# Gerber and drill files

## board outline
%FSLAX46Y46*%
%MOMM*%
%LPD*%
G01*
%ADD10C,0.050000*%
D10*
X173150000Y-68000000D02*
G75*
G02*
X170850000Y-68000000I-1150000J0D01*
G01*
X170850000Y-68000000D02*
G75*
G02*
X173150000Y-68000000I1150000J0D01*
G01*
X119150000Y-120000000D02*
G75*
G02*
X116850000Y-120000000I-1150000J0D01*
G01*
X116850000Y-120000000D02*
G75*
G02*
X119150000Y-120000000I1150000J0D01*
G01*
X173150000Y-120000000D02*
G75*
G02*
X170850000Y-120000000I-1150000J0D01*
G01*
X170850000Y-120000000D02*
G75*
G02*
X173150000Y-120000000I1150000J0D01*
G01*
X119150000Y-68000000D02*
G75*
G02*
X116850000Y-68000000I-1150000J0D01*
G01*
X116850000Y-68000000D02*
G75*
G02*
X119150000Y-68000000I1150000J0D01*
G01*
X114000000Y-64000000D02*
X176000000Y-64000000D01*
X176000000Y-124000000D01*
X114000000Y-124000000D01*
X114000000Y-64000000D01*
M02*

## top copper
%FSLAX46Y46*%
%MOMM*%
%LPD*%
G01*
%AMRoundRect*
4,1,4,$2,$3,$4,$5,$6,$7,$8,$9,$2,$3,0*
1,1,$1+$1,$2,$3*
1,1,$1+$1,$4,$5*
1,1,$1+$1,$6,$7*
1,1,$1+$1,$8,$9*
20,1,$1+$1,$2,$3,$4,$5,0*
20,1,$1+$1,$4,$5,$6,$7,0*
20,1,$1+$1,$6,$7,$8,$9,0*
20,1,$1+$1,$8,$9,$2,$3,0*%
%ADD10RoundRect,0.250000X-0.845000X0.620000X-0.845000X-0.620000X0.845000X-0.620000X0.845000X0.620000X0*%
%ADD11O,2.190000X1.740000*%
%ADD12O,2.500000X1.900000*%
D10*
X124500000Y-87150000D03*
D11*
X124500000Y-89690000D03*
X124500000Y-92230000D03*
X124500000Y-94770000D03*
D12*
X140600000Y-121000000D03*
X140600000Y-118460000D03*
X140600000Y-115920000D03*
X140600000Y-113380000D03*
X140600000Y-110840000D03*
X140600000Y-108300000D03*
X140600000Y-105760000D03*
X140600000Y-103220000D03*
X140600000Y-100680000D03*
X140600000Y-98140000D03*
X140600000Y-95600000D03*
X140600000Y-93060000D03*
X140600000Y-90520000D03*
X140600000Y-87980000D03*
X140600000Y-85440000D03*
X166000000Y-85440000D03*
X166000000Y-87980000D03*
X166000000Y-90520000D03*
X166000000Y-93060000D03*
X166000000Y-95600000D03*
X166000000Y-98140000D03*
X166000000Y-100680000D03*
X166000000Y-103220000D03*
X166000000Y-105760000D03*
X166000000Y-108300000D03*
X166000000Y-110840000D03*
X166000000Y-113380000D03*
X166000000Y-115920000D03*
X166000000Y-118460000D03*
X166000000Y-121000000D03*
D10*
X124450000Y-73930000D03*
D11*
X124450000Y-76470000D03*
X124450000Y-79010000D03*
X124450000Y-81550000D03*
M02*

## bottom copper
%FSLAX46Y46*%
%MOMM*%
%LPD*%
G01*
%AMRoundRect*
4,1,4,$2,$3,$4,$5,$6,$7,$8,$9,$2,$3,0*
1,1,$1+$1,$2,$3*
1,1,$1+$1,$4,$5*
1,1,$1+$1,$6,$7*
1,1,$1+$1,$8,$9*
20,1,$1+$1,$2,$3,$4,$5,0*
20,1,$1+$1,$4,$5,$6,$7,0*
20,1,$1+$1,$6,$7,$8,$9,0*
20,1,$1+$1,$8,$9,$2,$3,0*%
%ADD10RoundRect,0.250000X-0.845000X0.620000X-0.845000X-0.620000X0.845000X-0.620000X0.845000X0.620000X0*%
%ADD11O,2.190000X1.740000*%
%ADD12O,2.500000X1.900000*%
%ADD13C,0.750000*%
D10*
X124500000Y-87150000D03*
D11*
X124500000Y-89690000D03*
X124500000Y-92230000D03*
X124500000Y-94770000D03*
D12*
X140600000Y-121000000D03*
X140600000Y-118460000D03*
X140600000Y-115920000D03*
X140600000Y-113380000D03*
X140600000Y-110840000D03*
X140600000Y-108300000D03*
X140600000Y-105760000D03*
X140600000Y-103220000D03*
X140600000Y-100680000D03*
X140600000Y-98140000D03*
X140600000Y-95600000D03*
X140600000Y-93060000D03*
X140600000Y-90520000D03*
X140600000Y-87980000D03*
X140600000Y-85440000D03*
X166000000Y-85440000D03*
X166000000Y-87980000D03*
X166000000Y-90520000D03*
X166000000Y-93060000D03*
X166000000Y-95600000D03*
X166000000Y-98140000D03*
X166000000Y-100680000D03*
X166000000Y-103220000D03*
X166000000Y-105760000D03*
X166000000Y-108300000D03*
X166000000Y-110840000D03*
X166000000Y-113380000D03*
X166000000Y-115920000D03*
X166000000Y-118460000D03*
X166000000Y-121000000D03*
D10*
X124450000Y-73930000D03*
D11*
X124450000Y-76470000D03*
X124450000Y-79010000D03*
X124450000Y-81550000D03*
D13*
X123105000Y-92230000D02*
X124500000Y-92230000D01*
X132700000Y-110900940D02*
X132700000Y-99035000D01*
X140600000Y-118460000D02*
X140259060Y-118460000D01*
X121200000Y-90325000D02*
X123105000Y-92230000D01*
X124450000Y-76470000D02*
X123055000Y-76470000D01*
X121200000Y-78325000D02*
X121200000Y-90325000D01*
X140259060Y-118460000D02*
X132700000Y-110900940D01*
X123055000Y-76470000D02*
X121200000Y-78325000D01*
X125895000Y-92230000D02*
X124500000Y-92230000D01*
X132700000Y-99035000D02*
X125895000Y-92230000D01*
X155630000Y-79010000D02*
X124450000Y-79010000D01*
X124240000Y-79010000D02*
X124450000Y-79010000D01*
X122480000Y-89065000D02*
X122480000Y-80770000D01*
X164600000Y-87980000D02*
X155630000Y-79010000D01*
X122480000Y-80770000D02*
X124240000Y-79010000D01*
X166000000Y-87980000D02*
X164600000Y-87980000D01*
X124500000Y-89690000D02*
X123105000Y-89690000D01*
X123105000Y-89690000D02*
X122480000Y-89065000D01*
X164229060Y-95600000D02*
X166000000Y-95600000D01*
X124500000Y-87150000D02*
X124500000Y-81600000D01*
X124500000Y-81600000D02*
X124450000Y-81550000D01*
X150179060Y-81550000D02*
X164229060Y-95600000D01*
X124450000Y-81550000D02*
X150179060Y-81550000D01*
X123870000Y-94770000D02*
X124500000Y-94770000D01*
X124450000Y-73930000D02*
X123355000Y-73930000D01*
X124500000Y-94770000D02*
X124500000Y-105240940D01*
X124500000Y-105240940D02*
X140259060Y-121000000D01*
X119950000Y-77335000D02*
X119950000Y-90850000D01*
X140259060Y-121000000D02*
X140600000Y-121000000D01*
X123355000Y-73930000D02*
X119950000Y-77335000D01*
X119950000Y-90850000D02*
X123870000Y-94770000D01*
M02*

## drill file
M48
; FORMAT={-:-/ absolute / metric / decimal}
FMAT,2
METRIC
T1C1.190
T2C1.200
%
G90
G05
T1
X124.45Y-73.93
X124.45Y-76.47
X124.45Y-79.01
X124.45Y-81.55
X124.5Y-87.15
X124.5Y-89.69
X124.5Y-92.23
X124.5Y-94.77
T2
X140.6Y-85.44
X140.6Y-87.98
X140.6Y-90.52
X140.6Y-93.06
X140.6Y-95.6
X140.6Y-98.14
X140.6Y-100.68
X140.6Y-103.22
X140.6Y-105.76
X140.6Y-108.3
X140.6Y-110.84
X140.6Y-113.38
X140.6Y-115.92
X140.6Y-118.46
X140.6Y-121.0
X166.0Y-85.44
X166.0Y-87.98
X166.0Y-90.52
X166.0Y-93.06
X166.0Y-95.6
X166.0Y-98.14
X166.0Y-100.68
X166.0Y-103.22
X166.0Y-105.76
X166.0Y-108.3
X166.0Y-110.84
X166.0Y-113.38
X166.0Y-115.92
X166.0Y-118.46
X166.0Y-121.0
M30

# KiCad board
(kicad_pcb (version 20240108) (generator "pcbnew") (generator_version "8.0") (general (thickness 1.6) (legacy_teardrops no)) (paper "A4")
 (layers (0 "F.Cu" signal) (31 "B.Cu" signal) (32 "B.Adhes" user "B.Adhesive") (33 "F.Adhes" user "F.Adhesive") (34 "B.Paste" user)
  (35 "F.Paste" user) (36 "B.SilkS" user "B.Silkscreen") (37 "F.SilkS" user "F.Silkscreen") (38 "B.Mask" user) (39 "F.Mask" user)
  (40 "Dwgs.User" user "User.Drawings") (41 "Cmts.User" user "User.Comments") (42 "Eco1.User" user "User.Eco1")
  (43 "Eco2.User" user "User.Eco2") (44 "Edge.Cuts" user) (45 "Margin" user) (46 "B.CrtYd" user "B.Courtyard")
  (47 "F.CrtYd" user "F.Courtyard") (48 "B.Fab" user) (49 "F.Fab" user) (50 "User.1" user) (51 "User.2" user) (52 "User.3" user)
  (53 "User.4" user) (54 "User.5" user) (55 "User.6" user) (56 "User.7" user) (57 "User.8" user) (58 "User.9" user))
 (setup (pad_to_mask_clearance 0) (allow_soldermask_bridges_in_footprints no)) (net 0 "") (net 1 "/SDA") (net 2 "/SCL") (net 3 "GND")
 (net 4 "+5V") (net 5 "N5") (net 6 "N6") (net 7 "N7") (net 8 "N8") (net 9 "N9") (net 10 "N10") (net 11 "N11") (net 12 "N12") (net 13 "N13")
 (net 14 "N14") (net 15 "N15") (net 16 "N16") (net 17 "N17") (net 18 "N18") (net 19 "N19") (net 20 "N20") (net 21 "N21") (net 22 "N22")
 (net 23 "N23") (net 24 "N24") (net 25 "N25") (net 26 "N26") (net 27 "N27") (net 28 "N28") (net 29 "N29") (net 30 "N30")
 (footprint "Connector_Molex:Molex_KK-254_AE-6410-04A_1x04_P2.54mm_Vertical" (layer "F.Cu") (at 124.5 87.15 -90)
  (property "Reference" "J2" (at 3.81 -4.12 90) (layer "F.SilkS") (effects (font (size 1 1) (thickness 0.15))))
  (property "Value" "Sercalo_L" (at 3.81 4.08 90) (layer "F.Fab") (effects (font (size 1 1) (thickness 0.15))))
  (pad "1" thru_hole roundrect (at 0 0 270) (size 1.74 2.19) (drill 1.19) (layers "*.Cu" "*.Mask") (remove_unused_layers no)
   (roundrect_rratio 0.143678) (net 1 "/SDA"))
  (pad "2" thru_hole oval (at 2.54 0 270) (size 1.74 2.19) (drill 1.19) (layers "*.Cu" "*.Mask") (remove_unused_layers no) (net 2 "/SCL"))
  (pad "3" thru_hole oval (at 5.08 0 270) (size 1.74 2.19) (drill 1.19) (layers "*.Cu" "*.Mask") (remove_unused_layers no) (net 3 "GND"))
  (pad "4" thru_hole oval (at 7.62 0 270) (size 1.74 2.19) (drill 1.19) (layers "*.Cu" "*.Mask") (remove_unused_layers no) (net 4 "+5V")))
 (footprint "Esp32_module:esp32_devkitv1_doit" (layer "F.Cu") (at 153.3 104.49)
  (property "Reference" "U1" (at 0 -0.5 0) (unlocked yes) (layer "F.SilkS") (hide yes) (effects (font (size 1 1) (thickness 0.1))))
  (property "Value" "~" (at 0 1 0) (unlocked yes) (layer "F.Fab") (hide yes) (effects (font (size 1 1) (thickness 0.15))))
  (pad "1" thru_hole oval (at -12.7 16.51 180) (size 2.5 1.9) (drill 1.2) (layers "*.Cu" "*.Mask") (remove_unused_layers no) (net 4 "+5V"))
  (pad "2" thru_hole oval (at -12.7 13.97 180) (size 2.5 1.9) (drill 1.2) (layers "*.Cu" "*.Mask") (remove_unused_layers no) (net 3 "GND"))
  (pad "3" thru_hole oval (at -12.7 11.43 180) (size 2.5 1.9) (drill 1.2) (layers "*.Cu" "*.Mask") (remove_unused_layers no) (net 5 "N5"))
  (pad "4" thru_hole oval (at -12.7 8.89 180) (size 2.5 1.9) (drill 1.2) (layers "*.Cu" "*.Mask") (remove_unused_layers no) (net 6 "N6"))
  (pad "5" thru_hole oval (at -12.7 6.35 180) (size 2.5 1.9) (drill 1.2) (layers "*.Cu" "*.Mask") (remove_unused_layers no) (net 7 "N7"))
  (pad "6" thru_hole oval (at -12.7 3.81 180) (size 2.5 1.9) (drill 1.2) (layers "*.Cu" "*.Mask") (remove_unused_layers no) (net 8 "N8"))
  (pad "7" thru_hole oval (at -12.7 1.27 180) (size 2.5 1.9) (drill 1.2) (layers "*.Cu" "*.Mask") (remove_unused_layers no) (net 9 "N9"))
  (pad "8" thru_hole oval (at -12.7 -1.27 180) (size 2.5 1.9) (drill 1.2) (layers "*.Cu" "*.Mask") (remove_unused_layers no) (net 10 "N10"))
  (pad "9" thru_hole oval (at -12.7 -3.81 180) (size 2.5 1.9) (drill 1.2) (layers "*.Cu" "*.Mask") (remove_unused_layers no) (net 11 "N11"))
  (pad "10" thru_hole oval (at -12.7 -6.35 180) (size 2.5 1.9) (drill 1.2) (layers "*.Cu" "*.Mask") (remove_unused_layers no) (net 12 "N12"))
  (pad "11" thru_hole oval (at -12.7 -8.89 180) (size 2.5 1.9) (drill 1.2) (layers "*.Cu" "*.Mask") (remove_unused_layers no) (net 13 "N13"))
  (pad "12" thru_hole oval (at -12.7 -11.43 180) (size 2.5 1.9) (drill 1.2) (layers "*.Cu" "*.Mask") (remove_unused_layers no)
   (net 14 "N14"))
  (pad "13" thru_hole oval (at -12.7 -13.97 180) (size 2.5 1.9) (drill 1.2) (layers "*.Cu" "*.Mask") (remove_unused_layers no)
   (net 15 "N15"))
  (pad "14" thru_hole oval (at -12.7 -16.51 180) (size 2.5 1.9) (drill 1.2) (layers "*.Cu" "*.Mask") (remove_unused_layers no)
   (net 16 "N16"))
  (pad "15" thru_hole oval (at -12.7 -19.05 180) (size 2.5 1.9) (drill 1.2) (layers "*.Cu" "*.Mask") (remove_unused_layers no)
   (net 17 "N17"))
  (pad "16" thru_hole oval (at 12.7 -19.05 180) (size 2.5 1.9) (drill 1.2) (layers "*.Cu" "*.Mask") (remove_unused_layers no) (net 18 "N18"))
  (pad "17" thru_hole oval (at 12.7 -16.51 180) (size 2.5 1.9) (drill 1.2) (layers "*.Cu" "*.Mask") (remove_unused_layers no) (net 2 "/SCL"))
  (pad "18" thru_hole oval (at 12.7 -13.97 180) (size 2.5 1.9) (drill 1.2) (layers "*.Cu" "*.Mask") (remove_unused_layers no) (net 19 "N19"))
  (pad "19" thru_hole oval (at 12.7 -11.43 180) (size 2.5 1.9) (drill 1.2) (layers "*.Cu" "*.Mask") (remove_unused_layers no) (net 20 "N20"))
  (pad "20" thru_hole oval (at 12.7 -8.89 180) (size 2.5 1.9) (drill 1.2) (layers "*.Cu" "*.Mask") (remove_unused_layers no) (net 1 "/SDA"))
  (pad "21" thru_hole oval (at 12.7 -6.35 180) (size 2.5 1.9) (drill 1.2) (layers "*.Cu" "*.Mask") (remove_unused_layers no) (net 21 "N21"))
  (pad "22" thru_hole oval (at 12.7 -3.81 180) (size 2.5 1.9) (drill 1.2) (layers "*.Cu" "*.Mask") (remove_unused_layers no) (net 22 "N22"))
  (pad "23" thru_hole oval (at 12.7 -1.27 180) (size 2.5 1.9) (drill 1.2) (layers "*.Cu" "*.Mask") (remove_unused_layers no) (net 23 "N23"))
  (pad "24" thru_hole oval (at 12.7 1.27 180) (size 2.5 1.9) (drill 1.2) (layers "*.Cu" "*.Mask") (remove_unused_layers no) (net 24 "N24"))
  (pad "25" thru_hole oval (at 12.7 3.81 180) (size 2.5 1.9) (drill 1.2) (layers "*.Cu" "*.Mask") (remove_unused_layers no) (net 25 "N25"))
  (pad "26" thru_hole oval (at 12.7 6.35 180) (size 2.5 1.9) (drill 1.2) (layers "*.Cu" "*.Mask") (remove_unused_layers no) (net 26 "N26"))
  (pad "27" thru_hole oval (at 12.7 8.89 180) (size 2.5 1.9) (drill 1.2) (layers "*.Cu" "*.Mask") (remove_unused_layers no) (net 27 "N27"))
  (pad "28" thru_hole oval (at 12.7 11.43 180) (size 2.5 1.9) (drill 1.2) (layers "*.Cu" "*.Mask") (remove_unused_layers no) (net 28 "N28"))
  (pad "29" thru_hole oval (at 12.7 13.97 180) (size 2.5 1.9) (drill 1.2) (layers "*.Cu" "*.Mask") (remove_unused_layers no) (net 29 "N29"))
  (pad "30" thru_hole oval (at 12.7 16.51 180) (size 2.5 1.9) (drill 1.2) (layers "*.Cu" "*.Mask") (remove_unused_layers no) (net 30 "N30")))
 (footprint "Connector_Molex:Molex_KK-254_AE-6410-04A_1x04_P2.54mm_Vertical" (layer "F.Cu") (at 124.45 73.93 -90)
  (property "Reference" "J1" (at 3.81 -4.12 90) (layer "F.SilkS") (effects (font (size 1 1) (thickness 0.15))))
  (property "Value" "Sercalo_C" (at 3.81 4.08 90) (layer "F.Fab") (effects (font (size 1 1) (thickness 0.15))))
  (pad "1" thru_hole roundrect (at 0 0 270) (size 1.74 2.19) (drill 1.19) (layers "*.Cu" "*.Mask") (remove_unused_layers no)
   (roundrect_rratio 0.143678) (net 4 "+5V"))
  (pad "2" thru_hole oval (at 2.54 0 270) (size 1.74 2.19) (drill 1.19) (layers "*.Cu" "*.Mask") (remove_unused_layers no) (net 3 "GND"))
  (pad "3" thru_hole oval (at 5.08 0 270) (size 1.74 2.19) (drill 1.19) (layers "*.Cu" "*.Mask") (remove_unused_layers no) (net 2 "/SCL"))
  (pad "4" thru_hole oval (at 7.62 0 270) (size 1.74 2.19) (drill 1.19) (layers "*.Cu" "*.Mask") (remove_unused_layers no) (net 1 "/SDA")))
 (gr_circle (center 172 68) (end 173.15 68) (stroke (width 0.05) (type default)) (fill none) (layer "Edge.Cuts"))
 (gr_circle (center 118 120) (end 116.85 120) (stroke (width 0.05) (type default)) (fill none) (layer "Edge.Cuts"))
 (gr_circle (center 172 120) (end 173.15 120) (stroke (width 0.05) (type default)) (fill none) (layer "Edge.Cuts"))
 (gr_circle (center 118 68) (end 119.15 68) (stroke (width 0.05) (type default)) (fill none) (layer "Edge.Cuts"))
 (gr_rect (start 114 64) (end 176 124) (stroke (width 0.05) (type default)) (fill none) (layer "Edge.Cuts"))
 (segment (start 123.105 92.23) (end 124.5 92.23) (width 0.75) (layer "B.Cu") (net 3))
 (segment (start 132.7 110.90094) (end 132.7 99.035) (width 0.75) (layer "B.Cu") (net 3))
 (segment (start 140.6 118.46) (end 140.25906 118.46) (width 0.75) (layer "B.Cu") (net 3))
 (segment (start 121.2 90.325) (end 123.105 92.23) (width 0.75) (layer "B.Cu") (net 3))
 (segment (start 124.45 76.47) (end 123.055 76.47) (width 0.75) (layer "B.Cu") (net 3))
 (segment (start 121.2 78.325) (end 121.2 90.325) (width 0.75) (layer "B.Cu") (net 3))
 (segment (start 140.25906 118.46) (end 132.7 110.90094) (width 0.75) (layer "B.Cu") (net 3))
 (segment (start 123.055 76.47) (end 121.2 78.325) (width 0.75) (layer "B.Cu") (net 3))
 (segment (start 125.895 92.23) (end 124.5 92.23) (width 0.75) (layer "B.Cu") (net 3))
 (segment (start 132.7 99.035) (end 125.895 92.23) (width 0.75) (layer "B.Cu") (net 3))
 (segment (start 155.63 79.01) (end 124.45 79.01) (width 0.75) (layer "B.Cu") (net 2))
 (segment (start 124.24 79.01) (end 124.45 79.01) (width 0.75) (layer "B.Cu") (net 2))
 (segment (start 122.48 89.065) (end 122.48 80.77) (width 0.75) (layer "B.Cu") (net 2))
 (segment (start 164.6 87.98) (end 155.63 79.01) (width 0.75) (layer "B.Cu") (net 2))
 (segment (start 122.48 80.77) (end 124.24 79.01) (width 0.75) (layer "B.Cu") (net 2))
 (segment (start 166 87.98) (end 164.6 87.98) (width 0.75) (layer "B.Cu") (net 2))
 (segment (start 124.5 89.69) (end 123.105 89.69) (width 0.75) (layer "B.Cu") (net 2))
 (segment (start 123.105 89.69) (end 122.48 89.065) (width 0.75) (layer "B.Cu") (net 2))
 (segment (start 164.22906 95.6) (end 166 95.6) (width 0.75) (layer "B.Cu") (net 1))
 (segment (start 124.5 87.15) (end 124.5 81.6) (width 0.75) (layer "B.Cu") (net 1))
 (segment (start 124.5 81.6) (end 124.45 81.55) (width 0.75) (layer "B.Cu") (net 1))
 (segment (start 150.17906 81.55) (end 164.22906 95.6) (width 0.75) (layer "B.Cu") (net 1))
 (segment (start 124.45 81.55) (end 150.17906 81.55) (width 0.75) (layer "B.Cu") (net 1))
 (segment (start 123.87 94.77) (end 124.5 94.77) (width 0.75) (layer "B.Cu") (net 4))
 (segment (start 124.45 73.93) (end 123.355 73.93) (width 0.75) (layer "B.Cu") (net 4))
 (segment (start 124.5 94.77) (end 124.5 105.24094) (width 0.75) (layer "B.Cu") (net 4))
 (segment (start 124.5 105.24094) (end 140.25906 121) (width 0.75) (layer "B.Cu") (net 4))
 (segment (start 119.95 77.335) (end 119.95 90.85) (width 0.75) (layer "B.Cu") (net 4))
 (segment (start 140.25906 121) (end 140.6 121) (width 0.75) (layer "B.Cu") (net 4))
 (segment (start 123.355 73.93) (end 119.95 77.335) (width 0.75) (layer "B.Cu") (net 4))
 (segment (start 119.95 90.85) (end 123.87 94.77) (width 0.75) (layer "B.Cu") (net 4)))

